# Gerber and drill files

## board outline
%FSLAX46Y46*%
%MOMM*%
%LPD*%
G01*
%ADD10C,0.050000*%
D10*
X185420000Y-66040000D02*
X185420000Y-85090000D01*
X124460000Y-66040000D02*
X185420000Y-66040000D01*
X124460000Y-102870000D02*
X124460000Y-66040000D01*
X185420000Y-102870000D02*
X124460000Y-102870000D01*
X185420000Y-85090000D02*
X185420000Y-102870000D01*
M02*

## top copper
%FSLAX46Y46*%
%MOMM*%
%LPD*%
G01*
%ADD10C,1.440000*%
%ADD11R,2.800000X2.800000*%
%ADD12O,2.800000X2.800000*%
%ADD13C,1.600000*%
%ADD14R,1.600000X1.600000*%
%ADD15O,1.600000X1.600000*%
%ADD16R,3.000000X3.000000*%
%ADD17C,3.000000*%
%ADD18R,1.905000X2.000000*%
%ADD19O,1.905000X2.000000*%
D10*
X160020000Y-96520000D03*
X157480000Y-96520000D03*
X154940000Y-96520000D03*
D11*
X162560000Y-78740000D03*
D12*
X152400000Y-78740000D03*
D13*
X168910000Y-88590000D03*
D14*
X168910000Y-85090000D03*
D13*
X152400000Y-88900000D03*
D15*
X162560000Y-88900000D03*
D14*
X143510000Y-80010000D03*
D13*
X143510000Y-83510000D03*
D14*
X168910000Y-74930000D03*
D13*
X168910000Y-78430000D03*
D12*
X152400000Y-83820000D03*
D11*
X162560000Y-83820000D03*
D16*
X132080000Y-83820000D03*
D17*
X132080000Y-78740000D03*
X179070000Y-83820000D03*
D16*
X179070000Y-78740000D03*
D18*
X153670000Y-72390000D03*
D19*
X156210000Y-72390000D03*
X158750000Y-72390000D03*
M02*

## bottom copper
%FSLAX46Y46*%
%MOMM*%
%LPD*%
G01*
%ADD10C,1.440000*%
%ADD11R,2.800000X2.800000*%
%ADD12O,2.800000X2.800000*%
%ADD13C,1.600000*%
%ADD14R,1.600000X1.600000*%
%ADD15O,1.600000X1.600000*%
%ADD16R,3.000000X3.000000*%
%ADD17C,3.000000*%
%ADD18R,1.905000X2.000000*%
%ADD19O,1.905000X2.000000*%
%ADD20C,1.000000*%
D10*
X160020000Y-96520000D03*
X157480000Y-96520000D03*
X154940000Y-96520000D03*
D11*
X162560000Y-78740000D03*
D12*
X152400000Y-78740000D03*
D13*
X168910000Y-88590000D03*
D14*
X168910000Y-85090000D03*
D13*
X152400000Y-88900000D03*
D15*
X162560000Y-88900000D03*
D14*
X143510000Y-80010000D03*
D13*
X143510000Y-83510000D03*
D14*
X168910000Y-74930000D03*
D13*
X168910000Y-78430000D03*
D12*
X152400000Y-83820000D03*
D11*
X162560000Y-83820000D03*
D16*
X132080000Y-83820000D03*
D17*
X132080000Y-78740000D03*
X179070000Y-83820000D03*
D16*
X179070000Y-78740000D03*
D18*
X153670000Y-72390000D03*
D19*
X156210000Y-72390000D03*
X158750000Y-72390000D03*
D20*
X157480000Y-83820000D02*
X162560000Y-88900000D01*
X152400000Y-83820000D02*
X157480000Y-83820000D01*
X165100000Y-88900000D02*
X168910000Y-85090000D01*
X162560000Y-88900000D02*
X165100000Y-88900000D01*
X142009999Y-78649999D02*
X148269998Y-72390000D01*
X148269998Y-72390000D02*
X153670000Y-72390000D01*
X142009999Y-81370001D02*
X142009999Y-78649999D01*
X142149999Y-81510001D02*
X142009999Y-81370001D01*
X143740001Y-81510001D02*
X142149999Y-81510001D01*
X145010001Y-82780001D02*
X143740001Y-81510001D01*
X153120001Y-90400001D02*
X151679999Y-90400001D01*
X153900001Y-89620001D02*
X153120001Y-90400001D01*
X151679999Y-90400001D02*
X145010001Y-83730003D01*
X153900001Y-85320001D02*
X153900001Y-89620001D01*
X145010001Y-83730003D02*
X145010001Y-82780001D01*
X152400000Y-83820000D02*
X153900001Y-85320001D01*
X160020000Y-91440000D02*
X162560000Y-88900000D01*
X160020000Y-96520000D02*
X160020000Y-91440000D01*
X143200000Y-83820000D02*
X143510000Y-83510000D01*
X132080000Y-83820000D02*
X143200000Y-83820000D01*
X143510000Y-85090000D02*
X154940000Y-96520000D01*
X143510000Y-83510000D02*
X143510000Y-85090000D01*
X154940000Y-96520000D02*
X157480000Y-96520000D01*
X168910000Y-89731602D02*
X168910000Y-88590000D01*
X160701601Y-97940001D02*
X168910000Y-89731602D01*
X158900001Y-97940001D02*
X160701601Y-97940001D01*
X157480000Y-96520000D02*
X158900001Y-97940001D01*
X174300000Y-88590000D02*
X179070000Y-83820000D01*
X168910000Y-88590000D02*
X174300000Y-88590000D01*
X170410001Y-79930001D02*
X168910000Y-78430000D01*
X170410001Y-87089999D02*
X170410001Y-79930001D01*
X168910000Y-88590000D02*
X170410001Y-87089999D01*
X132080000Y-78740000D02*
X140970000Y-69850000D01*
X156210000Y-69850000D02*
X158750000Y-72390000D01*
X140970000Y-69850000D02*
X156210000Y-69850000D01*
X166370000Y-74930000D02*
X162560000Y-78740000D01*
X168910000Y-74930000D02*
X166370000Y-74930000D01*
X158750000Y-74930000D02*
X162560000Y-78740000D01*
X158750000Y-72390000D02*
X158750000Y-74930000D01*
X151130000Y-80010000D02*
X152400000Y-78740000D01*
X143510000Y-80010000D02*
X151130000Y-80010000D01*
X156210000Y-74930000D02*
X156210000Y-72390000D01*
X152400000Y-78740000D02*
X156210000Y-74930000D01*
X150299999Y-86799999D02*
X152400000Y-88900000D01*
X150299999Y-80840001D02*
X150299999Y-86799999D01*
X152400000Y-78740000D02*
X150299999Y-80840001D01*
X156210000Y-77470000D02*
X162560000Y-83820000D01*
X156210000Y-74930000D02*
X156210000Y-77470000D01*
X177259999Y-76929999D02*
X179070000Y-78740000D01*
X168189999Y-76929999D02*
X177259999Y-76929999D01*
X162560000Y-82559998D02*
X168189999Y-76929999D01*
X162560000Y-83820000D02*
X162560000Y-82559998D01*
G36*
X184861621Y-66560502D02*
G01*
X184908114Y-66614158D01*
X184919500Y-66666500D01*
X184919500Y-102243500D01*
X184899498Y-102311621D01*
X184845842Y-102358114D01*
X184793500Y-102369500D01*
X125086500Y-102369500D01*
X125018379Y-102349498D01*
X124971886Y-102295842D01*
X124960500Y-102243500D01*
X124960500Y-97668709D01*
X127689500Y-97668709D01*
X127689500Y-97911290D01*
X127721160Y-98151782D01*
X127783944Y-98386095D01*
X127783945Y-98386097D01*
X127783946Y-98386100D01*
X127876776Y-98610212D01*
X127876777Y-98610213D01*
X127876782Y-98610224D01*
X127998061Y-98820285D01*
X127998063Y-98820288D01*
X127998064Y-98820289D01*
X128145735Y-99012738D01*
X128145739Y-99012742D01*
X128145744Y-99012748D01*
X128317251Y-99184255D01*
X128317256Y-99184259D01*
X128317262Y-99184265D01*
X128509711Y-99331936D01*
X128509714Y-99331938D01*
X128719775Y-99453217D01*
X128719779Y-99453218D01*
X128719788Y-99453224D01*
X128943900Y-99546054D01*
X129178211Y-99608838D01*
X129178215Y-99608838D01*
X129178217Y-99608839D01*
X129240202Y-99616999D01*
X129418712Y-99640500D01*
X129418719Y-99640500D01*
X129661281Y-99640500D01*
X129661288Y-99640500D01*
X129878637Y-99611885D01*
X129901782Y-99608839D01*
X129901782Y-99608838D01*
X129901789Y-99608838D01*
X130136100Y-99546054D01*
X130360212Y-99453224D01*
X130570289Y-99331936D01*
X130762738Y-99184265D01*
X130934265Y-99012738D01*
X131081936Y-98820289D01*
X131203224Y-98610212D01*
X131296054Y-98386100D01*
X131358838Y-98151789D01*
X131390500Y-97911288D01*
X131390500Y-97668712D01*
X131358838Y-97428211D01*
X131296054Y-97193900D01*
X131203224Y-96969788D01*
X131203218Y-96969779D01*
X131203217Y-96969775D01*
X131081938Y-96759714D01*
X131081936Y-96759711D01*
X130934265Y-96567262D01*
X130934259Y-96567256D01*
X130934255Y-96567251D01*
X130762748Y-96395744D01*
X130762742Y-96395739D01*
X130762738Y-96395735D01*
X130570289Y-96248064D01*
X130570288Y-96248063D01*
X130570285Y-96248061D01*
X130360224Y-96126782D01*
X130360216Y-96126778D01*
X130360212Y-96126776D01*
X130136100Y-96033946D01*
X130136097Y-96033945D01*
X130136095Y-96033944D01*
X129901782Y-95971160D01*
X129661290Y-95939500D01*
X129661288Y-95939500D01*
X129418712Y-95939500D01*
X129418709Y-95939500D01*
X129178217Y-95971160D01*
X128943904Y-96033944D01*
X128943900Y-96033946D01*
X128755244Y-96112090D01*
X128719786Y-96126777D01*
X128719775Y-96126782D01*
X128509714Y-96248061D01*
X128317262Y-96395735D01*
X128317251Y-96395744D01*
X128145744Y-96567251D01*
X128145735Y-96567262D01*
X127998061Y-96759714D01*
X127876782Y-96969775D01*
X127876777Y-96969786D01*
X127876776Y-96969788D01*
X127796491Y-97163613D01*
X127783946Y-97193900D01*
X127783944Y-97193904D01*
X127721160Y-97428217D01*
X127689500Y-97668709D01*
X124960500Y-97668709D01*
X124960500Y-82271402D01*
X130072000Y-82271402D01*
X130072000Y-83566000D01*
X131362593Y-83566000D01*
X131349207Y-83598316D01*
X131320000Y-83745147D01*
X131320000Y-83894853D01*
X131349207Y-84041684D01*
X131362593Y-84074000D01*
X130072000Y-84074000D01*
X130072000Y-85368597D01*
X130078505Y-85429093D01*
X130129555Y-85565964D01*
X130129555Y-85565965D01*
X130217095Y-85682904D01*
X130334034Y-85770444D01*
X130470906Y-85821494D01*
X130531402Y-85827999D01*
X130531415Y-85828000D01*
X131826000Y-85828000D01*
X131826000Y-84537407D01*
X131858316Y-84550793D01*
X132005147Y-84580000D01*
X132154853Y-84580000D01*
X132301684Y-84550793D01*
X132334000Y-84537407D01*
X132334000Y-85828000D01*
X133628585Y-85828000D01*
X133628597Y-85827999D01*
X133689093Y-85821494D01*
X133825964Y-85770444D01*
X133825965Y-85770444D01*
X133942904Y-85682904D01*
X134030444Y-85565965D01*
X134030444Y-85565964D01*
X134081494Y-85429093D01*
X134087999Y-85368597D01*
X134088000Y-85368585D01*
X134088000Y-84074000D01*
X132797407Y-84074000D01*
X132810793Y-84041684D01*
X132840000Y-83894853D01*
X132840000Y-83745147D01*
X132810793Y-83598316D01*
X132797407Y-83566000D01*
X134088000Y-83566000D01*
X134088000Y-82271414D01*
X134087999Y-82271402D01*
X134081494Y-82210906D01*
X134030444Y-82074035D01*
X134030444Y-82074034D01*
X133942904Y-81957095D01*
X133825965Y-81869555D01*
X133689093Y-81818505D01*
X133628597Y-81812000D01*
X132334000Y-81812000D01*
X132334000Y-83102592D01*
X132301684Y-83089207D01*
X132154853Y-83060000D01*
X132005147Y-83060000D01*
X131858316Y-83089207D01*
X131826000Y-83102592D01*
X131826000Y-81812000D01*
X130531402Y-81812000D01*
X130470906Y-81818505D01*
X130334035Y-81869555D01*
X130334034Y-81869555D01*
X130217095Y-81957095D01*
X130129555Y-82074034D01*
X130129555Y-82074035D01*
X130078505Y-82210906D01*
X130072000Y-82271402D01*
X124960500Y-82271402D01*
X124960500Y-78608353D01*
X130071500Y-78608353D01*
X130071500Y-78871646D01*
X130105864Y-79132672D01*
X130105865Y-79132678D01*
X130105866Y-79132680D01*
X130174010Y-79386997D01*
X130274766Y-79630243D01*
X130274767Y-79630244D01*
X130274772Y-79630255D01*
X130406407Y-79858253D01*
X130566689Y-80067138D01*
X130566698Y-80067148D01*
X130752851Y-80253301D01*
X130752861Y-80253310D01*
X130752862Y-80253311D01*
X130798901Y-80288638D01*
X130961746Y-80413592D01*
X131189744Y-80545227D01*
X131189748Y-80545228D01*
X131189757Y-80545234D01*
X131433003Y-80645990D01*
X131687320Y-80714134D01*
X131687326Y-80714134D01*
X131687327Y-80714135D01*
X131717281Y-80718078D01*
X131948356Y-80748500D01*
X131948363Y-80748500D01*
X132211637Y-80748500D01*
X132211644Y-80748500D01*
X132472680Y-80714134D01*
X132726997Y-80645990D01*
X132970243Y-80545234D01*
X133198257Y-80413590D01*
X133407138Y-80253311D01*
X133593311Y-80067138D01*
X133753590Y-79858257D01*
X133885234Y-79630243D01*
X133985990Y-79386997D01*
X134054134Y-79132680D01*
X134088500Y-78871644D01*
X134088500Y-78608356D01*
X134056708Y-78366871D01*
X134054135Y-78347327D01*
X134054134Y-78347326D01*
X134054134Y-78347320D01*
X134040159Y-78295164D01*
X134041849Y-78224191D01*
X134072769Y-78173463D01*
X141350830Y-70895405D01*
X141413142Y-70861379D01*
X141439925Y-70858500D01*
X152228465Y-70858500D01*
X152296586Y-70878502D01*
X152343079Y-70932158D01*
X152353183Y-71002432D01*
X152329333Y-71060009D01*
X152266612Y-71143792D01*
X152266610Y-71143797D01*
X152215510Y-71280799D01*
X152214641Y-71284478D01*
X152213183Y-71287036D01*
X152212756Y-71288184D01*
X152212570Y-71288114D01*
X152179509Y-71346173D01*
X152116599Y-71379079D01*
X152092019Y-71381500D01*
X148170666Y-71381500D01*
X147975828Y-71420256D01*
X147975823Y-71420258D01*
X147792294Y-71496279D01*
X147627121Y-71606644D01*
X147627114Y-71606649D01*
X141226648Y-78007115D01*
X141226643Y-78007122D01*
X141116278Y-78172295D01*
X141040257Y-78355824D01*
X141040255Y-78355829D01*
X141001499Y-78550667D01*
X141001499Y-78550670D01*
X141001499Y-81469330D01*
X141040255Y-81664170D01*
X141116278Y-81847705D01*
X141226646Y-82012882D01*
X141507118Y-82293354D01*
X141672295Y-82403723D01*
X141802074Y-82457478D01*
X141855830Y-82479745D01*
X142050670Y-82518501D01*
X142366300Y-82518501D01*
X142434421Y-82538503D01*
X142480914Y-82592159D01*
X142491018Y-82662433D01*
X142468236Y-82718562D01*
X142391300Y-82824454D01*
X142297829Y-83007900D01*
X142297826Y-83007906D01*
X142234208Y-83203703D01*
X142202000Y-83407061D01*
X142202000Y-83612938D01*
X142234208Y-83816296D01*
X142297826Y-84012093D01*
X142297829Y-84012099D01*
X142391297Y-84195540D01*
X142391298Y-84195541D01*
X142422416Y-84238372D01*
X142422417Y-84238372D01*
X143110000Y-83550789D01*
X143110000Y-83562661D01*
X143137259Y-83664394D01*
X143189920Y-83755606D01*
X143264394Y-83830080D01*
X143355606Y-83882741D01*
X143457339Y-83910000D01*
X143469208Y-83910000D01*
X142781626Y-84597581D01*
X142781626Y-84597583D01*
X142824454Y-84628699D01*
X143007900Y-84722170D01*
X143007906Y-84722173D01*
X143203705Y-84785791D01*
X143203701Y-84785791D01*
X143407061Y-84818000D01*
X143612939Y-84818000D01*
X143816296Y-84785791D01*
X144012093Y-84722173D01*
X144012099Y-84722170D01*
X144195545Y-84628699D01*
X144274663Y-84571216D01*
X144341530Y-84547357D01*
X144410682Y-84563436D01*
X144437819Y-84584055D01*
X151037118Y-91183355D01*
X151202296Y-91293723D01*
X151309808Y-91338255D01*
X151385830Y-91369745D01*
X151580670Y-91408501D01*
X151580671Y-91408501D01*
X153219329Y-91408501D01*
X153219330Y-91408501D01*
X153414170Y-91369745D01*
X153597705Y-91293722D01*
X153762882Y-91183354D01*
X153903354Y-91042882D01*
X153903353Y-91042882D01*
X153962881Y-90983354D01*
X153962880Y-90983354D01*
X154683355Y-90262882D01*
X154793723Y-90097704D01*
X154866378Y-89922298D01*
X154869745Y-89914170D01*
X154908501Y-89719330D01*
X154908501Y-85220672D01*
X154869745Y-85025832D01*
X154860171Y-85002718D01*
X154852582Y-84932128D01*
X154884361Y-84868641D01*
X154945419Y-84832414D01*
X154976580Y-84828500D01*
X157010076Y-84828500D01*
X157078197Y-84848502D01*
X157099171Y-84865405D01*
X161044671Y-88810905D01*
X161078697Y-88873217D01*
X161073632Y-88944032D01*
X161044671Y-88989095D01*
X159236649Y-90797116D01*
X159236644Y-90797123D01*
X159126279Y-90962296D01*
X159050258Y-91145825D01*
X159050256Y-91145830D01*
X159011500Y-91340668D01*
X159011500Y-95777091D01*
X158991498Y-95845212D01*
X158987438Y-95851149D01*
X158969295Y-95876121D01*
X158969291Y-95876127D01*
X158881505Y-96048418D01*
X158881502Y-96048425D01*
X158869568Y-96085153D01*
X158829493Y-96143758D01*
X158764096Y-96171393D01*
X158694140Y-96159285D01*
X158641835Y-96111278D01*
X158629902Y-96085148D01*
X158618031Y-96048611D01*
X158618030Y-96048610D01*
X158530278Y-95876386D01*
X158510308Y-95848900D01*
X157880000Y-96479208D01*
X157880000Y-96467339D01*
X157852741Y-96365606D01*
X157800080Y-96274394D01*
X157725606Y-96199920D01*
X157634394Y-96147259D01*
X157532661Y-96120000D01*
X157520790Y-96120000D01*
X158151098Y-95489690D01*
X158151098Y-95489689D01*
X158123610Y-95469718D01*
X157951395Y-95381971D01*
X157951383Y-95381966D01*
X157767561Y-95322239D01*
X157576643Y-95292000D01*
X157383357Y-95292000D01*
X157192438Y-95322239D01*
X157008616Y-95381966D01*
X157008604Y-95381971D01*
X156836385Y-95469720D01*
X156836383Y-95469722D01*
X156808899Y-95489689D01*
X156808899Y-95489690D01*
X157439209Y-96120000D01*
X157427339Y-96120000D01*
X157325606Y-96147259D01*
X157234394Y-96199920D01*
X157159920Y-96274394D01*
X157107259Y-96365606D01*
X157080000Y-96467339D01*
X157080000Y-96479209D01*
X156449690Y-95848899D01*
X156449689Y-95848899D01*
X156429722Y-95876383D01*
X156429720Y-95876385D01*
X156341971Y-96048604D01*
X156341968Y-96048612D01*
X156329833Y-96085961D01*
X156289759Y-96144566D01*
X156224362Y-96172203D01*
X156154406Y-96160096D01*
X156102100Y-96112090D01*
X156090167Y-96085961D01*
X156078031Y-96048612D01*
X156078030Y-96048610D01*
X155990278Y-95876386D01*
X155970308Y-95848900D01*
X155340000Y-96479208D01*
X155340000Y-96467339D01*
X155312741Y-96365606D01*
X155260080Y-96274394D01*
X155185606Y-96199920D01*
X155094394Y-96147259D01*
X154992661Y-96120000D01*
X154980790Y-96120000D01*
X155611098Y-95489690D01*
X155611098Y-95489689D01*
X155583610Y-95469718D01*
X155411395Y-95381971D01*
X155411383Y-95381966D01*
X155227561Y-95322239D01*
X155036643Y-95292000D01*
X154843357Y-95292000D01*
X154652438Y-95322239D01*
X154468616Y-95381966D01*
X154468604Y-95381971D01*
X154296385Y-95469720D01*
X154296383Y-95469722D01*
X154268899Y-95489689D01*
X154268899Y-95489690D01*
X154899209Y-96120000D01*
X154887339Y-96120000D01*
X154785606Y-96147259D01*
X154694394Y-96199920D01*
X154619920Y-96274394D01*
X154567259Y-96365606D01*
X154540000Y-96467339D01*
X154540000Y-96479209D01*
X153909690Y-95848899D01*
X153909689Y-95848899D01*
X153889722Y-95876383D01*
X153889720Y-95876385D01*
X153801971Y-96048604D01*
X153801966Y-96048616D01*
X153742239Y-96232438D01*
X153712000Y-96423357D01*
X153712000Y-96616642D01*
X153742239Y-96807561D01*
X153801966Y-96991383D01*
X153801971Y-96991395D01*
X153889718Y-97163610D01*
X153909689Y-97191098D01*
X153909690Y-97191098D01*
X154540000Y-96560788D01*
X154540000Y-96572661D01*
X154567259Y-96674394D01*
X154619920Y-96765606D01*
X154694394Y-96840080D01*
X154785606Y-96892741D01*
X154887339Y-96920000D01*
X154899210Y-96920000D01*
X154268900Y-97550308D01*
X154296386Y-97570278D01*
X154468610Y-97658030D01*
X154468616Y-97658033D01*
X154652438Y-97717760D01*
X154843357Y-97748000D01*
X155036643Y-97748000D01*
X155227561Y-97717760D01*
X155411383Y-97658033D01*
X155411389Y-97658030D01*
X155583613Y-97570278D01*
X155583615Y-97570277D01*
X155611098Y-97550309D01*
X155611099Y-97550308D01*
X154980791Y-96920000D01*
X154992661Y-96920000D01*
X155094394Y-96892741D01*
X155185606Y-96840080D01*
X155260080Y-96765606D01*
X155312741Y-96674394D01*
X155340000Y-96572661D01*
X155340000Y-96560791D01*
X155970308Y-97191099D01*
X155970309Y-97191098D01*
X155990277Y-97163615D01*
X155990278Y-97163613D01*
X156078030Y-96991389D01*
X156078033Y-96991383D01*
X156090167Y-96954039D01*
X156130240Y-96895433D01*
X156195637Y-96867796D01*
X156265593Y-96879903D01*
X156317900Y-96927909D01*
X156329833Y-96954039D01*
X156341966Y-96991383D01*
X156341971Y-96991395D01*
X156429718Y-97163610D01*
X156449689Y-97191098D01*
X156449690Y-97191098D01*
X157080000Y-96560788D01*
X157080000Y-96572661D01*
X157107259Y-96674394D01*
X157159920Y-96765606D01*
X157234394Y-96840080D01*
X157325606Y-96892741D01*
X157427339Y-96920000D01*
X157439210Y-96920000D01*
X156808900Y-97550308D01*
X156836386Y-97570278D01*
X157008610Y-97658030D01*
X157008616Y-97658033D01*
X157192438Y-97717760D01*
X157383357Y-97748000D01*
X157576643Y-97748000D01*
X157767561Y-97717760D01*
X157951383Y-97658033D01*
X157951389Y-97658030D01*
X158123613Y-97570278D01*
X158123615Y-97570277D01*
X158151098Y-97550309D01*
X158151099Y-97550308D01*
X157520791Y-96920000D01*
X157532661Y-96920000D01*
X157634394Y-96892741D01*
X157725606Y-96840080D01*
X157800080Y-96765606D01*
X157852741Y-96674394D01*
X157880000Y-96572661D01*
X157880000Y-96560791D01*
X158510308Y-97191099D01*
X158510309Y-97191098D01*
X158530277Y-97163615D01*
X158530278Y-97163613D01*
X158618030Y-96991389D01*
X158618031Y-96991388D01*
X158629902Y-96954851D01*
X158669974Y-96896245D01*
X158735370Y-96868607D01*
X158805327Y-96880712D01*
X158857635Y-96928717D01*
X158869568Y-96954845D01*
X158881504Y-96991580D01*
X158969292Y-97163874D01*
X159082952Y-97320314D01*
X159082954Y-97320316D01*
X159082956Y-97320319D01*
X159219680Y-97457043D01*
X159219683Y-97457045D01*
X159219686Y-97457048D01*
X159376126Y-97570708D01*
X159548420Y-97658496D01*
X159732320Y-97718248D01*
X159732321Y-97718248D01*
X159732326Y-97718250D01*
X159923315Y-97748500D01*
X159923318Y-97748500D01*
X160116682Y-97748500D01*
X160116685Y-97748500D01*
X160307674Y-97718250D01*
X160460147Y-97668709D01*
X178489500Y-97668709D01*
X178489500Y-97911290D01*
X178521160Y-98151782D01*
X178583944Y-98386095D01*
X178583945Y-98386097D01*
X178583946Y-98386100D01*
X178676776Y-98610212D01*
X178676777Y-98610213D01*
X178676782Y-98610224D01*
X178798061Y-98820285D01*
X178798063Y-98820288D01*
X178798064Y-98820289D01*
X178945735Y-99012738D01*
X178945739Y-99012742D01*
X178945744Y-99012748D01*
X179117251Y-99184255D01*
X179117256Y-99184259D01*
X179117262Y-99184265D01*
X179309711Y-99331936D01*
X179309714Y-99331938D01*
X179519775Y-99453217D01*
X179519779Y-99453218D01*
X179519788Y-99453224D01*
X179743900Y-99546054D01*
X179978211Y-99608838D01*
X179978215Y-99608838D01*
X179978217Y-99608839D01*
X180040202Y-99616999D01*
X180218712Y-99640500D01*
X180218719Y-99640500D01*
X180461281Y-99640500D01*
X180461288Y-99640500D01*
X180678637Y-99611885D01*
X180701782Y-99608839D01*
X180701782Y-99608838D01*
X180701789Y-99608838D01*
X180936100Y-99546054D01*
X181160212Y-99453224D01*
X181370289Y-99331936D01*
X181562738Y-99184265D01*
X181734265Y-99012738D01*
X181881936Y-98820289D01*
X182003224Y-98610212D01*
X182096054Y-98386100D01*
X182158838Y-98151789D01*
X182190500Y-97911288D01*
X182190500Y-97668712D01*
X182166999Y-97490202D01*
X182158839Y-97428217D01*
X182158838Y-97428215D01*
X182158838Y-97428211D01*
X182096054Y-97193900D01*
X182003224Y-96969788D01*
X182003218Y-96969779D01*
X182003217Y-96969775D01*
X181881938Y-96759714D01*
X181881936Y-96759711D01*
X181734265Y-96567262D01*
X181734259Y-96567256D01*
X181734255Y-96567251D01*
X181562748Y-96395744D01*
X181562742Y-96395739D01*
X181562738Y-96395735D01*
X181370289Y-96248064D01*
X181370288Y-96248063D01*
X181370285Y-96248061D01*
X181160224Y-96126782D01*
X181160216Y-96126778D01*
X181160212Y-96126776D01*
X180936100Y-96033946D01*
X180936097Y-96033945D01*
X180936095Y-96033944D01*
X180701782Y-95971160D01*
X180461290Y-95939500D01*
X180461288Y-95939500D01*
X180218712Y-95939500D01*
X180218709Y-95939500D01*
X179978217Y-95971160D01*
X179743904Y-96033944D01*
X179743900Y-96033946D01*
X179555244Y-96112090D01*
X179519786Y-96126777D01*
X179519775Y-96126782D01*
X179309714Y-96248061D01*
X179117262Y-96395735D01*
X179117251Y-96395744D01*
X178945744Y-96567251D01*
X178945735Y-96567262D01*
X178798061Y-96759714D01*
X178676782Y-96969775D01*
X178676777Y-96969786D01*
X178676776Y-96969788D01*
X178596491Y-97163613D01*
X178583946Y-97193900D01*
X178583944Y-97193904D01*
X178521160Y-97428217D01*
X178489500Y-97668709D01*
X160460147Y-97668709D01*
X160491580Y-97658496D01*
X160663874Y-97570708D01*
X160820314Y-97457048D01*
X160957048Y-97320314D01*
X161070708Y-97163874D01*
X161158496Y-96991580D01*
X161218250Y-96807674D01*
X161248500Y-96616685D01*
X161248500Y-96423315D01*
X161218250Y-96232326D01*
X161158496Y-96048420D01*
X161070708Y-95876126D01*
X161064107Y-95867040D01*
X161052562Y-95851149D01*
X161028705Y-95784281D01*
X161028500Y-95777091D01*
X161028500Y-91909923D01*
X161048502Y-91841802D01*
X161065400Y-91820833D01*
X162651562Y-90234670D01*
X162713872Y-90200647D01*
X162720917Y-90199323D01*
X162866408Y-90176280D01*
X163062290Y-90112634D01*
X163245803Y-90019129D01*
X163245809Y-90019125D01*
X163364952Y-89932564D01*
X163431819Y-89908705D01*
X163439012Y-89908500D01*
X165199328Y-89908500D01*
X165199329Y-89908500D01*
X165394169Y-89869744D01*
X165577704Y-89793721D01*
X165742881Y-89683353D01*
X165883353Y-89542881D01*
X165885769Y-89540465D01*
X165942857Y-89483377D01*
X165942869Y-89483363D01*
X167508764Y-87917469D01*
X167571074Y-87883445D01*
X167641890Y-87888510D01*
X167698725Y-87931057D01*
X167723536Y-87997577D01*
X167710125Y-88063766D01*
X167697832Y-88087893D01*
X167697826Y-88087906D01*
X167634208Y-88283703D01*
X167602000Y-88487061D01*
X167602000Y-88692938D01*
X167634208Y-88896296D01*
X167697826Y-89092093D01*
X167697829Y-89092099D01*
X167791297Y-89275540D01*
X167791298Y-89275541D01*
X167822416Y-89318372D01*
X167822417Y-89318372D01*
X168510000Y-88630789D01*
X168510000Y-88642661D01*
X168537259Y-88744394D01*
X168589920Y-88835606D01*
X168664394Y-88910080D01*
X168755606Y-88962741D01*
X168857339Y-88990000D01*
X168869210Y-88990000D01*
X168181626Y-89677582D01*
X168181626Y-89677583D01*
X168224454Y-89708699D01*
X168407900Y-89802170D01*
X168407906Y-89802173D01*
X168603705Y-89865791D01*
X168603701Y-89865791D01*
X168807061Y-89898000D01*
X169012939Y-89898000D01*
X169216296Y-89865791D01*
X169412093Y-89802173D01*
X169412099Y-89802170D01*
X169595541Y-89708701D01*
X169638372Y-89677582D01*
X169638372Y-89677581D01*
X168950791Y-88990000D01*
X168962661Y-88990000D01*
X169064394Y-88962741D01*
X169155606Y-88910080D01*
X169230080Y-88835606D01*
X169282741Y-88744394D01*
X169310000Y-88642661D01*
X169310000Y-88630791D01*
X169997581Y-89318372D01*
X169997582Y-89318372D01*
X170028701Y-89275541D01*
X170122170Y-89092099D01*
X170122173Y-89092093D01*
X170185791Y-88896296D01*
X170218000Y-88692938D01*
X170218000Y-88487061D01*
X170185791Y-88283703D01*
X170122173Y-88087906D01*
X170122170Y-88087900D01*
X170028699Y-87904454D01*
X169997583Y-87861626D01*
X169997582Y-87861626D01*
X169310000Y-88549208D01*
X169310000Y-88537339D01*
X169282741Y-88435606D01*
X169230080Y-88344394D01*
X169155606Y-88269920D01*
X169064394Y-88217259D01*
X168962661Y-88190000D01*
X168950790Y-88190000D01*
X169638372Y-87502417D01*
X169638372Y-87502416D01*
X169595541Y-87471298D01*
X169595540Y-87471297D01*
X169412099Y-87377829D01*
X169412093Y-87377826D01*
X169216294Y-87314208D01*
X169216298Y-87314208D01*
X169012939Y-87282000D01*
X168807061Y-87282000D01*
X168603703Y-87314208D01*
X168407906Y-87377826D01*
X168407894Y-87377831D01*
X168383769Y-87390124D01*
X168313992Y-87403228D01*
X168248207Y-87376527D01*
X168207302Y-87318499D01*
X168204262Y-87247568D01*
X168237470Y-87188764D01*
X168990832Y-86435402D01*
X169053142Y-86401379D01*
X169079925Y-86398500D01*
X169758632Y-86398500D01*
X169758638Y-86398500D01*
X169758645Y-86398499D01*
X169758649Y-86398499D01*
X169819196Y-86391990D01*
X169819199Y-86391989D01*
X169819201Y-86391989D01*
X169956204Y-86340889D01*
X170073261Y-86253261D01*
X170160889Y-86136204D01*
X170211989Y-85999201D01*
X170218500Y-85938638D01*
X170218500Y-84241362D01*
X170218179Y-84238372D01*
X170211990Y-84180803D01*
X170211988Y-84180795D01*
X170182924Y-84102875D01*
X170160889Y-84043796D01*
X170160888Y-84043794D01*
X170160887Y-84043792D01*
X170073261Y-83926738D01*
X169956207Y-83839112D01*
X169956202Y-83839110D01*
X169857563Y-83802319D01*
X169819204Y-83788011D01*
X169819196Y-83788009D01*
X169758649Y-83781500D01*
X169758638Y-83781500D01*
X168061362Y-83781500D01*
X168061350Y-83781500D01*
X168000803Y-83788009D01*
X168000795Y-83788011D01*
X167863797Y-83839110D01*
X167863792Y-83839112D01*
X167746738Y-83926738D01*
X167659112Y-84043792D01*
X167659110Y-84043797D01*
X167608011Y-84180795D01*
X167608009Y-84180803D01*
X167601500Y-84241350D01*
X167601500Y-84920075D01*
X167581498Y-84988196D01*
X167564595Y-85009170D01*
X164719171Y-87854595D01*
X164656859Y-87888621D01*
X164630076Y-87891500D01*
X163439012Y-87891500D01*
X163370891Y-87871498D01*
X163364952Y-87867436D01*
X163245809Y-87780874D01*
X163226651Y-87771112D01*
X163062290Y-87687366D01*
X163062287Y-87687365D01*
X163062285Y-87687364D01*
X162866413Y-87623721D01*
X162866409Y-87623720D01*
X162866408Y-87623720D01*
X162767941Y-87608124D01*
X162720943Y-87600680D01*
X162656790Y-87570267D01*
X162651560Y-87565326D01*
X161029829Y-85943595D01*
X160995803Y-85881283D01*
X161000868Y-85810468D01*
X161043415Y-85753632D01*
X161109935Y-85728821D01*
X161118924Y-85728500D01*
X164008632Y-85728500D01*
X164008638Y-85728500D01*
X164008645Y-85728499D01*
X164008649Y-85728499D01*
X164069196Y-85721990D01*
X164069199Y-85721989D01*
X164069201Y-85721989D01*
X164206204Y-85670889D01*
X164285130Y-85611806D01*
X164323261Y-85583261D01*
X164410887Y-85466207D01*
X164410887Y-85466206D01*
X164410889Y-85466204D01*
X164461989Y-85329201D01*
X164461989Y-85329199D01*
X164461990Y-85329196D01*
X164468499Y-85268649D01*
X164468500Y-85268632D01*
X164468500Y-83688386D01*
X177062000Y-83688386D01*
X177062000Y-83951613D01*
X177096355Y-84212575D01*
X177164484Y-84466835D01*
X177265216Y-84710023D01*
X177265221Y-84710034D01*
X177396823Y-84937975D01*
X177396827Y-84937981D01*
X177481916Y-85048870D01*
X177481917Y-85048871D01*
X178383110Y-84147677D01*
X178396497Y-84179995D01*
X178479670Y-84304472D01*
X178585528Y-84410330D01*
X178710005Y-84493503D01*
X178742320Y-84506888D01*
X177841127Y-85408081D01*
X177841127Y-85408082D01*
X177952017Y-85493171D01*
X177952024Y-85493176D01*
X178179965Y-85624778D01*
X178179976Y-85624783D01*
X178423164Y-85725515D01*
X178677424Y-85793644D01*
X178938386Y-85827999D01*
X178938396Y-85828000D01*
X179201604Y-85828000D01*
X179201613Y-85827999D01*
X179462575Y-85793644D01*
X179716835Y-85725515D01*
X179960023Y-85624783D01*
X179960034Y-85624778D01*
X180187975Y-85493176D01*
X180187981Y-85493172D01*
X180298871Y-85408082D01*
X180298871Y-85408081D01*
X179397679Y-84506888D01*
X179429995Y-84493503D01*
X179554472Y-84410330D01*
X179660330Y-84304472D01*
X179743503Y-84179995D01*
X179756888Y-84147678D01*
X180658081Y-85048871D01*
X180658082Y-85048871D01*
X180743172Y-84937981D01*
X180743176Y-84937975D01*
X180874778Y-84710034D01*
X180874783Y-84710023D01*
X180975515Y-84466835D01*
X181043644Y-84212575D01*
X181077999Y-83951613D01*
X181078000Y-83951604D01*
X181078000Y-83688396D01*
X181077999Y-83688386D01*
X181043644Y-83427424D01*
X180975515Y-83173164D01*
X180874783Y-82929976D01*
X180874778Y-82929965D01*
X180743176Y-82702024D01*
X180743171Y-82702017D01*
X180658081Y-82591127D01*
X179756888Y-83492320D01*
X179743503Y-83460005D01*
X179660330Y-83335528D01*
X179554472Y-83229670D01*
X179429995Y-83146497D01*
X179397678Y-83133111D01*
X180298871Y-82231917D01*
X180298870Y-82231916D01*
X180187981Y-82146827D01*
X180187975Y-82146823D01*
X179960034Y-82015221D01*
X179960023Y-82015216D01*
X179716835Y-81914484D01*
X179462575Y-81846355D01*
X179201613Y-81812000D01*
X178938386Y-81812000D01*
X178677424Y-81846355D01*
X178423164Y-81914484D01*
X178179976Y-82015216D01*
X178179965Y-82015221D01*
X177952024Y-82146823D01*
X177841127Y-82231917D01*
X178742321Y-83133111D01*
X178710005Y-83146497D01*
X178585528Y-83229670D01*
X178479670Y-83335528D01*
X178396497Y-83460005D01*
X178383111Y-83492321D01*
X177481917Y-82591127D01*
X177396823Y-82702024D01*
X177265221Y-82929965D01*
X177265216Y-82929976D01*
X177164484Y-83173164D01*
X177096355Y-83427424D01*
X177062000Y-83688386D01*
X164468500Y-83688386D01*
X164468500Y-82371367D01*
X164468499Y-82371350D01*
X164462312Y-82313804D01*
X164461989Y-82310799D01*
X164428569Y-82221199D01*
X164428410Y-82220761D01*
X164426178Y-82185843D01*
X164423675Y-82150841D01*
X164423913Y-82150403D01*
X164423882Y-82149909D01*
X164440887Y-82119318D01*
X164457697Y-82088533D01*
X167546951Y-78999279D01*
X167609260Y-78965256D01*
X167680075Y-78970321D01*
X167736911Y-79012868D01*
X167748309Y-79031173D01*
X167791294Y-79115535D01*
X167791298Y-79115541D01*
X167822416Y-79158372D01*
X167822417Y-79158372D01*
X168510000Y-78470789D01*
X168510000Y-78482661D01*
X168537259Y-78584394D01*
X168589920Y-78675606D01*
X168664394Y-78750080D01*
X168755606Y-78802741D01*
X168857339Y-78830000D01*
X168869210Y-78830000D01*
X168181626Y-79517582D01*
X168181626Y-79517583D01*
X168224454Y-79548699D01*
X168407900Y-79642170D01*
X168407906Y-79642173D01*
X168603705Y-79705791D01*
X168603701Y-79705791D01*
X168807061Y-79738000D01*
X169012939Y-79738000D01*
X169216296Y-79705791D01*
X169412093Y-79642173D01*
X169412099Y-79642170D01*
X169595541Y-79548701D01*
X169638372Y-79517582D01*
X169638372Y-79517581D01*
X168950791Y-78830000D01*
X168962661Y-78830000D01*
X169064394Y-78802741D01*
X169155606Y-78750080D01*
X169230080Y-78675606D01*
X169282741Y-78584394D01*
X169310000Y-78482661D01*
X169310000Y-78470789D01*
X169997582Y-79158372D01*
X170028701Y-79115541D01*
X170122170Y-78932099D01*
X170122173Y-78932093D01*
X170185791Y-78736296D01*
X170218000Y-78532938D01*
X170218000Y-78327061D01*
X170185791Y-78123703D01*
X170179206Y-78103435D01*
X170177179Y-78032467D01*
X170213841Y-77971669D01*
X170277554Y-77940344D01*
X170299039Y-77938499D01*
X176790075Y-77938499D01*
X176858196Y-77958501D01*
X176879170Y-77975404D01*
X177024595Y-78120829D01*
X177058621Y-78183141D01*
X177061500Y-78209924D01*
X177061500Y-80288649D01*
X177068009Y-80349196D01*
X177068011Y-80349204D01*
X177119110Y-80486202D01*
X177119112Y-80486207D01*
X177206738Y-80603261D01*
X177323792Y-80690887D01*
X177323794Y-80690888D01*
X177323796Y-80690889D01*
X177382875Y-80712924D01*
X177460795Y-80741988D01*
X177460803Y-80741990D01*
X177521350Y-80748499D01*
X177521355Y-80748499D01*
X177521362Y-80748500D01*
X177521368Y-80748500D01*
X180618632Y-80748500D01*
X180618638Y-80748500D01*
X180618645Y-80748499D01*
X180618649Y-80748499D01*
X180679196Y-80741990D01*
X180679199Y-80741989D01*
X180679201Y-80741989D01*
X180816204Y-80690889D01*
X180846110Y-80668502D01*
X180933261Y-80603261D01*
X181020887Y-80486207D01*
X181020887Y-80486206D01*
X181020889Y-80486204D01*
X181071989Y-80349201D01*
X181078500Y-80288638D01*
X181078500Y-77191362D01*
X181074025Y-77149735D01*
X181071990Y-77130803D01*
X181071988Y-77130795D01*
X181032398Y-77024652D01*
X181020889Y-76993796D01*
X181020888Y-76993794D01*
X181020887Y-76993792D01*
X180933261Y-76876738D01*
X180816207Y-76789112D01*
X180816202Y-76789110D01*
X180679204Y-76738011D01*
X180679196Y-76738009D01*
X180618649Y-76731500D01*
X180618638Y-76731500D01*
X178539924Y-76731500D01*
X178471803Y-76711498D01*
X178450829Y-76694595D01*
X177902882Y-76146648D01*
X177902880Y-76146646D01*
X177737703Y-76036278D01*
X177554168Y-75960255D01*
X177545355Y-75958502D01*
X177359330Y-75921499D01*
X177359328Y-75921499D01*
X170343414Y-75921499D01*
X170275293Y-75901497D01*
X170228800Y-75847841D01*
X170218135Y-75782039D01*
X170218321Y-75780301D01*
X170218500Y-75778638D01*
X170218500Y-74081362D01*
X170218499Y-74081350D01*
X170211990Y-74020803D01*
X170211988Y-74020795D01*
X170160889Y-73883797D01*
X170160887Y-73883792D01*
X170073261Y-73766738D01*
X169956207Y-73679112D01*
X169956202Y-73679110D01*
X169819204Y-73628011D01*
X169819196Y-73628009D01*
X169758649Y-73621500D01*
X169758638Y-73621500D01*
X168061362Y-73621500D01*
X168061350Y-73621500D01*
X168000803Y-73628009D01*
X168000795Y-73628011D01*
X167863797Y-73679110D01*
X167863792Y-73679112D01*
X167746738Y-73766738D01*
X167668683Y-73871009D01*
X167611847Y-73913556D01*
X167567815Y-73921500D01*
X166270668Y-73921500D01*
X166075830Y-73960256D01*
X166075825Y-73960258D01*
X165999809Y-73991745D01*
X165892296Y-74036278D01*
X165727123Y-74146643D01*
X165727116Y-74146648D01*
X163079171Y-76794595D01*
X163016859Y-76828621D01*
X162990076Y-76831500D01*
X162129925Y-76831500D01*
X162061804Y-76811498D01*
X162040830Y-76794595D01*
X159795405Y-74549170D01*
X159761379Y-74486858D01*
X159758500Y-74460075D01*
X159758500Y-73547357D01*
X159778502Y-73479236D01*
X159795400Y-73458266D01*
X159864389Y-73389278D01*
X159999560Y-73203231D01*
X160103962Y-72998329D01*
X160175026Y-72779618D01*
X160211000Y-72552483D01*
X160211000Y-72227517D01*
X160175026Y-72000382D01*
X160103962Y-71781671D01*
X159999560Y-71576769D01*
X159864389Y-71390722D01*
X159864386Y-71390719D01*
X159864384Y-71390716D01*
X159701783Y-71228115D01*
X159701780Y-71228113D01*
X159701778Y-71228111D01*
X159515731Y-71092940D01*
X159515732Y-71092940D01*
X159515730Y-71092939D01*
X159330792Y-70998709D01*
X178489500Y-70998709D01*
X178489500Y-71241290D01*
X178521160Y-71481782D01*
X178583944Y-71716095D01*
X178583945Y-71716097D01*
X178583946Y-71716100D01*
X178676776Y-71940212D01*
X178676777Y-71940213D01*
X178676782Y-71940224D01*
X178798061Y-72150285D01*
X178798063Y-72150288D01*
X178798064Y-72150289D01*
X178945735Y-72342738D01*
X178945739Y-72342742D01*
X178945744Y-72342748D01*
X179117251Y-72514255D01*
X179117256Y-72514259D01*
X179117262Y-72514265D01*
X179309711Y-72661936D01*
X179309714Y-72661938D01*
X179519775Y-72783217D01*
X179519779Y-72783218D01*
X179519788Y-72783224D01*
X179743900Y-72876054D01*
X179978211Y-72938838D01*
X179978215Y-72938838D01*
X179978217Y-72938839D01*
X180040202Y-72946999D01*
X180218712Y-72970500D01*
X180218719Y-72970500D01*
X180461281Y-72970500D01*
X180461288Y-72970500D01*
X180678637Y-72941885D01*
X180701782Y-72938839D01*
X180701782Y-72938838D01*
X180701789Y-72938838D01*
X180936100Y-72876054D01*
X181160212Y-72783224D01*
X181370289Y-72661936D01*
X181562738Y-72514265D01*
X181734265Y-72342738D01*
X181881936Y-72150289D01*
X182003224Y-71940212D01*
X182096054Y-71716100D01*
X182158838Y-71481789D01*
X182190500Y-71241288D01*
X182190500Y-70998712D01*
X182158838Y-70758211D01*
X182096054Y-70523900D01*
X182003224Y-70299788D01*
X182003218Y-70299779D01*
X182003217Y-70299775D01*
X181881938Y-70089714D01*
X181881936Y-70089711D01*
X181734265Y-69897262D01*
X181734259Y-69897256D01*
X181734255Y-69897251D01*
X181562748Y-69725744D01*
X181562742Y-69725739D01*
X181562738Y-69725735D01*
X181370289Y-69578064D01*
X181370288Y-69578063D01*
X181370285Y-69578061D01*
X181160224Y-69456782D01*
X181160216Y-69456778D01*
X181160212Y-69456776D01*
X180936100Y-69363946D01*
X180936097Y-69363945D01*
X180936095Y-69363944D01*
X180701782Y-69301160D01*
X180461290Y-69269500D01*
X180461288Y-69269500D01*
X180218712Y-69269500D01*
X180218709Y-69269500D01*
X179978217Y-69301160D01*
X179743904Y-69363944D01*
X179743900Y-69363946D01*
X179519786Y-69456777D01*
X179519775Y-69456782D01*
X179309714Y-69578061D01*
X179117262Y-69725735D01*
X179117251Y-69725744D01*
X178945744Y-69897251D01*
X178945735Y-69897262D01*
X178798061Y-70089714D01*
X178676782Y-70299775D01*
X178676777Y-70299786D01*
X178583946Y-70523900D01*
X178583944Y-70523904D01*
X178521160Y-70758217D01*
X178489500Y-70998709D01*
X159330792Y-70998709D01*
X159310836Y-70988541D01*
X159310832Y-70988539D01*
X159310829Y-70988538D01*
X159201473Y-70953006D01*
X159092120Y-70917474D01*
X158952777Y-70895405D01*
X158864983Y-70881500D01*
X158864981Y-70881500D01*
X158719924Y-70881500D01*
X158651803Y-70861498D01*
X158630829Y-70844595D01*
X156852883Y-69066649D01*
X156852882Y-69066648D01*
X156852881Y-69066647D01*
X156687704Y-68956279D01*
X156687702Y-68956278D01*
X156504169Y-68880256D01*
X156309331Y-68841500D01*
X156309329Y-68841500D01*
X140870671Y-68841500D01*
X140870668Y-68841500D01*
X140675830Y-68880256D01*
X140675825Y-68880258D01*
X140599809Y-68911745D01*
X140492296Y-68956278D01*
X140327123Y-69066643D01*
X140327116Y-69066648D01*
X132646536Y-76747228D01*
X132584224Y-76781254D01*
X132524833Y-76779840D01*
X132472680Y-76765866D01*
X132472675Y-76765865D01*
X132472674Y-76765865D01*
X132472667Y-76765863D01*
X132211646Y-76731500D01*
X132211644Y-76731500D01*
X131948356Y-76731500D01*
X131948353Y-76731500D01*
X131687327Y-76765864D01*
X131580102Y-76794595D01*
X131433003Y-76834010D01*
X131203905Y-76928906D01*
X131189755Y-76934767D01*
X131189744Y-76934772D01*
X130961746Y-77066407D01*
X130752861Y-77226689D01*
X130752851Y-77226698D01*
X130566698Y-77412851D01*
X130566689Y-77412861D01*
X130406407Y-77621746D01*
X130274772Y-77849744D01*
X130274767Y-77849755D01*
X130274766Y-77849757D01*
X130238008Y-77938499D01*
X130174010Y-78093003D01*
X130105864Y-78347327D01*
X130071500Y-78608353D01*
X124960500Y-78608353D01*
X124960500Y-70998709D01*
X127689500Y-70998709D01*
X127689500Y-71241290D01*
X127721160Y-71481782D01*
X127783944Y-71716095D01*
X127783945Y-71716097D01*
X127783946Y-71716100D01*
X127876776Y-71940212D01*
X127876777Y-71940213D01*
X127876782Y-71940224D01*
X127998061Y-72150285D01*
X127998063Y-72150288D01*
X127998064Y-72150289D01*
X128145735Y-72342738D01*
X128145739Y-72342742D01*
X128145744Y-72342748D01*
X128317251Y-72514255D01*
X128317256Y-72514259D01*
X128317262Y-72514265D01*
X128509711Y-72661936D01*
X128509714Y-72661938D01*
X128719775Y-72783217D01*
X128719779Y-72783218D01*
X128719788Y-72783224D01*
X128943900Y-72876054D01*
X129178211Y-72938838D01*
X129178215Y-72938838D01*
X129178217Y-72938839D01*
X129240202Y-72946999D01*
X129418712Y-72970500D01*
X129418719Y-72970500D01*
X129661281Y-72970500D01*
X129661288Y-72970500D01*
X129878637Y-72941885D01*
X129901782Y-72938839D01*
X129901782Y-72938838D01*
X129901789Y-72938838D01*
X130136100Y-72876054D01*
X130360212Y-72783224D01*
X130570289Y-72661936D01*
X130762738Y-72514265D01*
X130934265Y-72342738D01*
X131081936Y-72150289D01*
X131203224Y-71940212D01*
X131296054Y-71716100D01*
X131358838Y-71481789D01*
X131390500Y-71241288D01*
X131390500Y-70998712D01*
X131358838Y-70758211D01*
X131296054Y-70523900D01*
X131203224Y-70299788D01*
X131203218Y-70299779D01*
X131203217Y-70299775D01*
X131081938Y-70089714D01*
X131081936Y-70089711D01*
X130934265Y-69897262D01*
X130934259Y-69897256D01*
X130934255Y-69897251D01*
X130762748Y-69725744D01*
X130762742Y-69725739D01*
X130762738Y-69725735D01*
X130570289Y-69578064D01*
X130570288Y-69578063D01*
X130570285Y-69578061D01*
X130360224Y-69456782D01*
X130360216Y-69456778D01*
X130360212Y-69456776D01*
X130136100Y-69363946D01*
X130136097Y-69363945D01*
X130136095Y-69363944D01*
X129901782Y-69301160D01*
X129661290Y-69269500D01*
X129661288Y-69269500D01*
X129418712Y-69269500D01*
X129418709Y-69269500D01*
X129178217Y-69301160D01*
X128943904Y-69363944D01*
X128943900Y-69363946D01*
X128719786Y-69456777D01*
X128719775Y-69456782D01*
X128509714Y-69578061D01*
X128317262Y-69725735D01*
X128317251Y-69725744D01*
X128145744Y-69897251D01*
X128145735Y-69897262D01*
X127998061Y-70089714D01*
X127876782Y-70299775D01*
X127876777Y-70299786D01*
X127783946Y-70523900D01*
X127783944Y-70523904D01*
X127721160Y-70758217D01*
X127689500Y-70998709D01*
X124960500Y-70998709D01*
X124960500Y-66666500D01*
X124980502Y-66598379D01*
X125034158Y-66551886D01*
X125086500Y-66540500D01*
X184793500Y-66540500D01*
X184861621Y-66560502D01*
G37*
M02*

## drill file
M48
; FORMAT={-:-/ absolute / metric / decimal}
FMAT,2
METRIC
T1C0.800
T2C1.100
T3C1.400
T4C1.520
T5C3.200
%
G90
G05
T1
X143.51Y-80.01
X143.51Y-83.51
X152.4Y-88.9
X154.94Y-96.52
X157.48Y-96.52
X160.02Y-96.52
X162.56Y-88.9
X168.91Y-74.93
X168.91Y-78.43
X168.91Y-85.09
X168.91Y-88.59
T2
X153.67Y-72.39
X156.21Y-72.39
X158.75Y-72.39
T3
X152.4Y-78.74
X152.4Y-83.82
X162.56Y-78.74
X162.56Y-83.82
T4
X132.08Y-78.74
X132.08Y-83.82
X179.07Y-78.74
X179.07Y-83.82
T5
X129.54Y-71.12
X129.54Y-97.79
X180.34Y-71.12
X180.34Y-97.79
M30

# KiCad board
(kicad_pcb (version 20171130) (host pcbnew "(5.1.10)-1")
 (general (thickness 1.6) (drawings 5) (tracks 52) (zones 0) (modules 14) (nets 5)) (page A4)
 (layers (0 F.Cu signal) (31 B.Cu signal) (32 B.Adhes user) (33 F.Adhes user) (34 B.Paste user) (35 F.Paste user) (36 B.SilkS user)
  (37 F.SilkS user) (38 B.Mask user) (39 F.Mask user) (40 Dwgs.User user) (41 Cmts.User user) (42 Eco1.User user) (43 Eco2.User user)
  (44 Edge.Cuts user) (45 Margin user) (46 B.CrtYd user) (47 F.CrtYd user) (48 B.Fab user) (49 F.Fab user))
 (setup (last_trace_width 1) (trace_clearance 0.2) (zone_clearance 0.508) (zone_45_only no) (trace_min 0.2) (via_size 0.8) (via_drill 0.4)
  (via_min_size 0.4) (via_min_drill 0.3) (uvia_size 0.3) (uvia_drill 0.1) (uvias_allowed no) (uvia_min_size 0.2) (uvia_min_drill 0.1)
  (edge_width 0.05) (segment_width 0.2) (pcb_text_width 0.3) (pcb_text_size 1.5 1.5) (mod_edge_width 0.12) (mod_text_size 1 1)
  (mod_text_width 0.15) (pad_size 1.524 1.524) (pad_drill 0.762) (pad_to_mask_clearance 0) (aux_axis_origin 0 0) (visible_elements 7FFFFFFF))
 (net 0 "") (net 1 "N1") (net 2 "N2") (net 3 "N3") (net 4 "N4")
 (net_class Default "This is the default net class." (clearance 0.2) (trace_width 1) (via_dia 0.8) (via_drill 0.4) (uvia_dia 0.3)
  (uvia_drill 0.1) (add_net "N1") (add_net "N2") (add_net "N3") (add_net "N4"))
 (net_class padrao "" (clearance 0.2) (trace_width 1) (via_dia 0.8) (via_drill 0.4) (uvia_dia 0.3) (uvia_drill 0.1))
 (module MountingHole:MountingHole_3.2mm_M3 (layer F.Cu) (at 129.54 97.79)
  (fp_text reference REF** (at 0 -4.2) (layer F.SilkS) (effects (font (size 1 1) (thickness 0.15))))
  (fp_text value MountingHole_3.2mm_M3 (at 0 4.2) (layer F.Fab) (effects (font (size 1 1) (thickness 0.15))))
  (pad 1 np_thru_hole circle (at 0 0) (size 3.2 3.2) (drill 3.2) (layers *.Cu *.Mask)))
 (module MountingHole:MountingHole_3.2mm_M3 (layer F.Cu) (at 129.54 71.12)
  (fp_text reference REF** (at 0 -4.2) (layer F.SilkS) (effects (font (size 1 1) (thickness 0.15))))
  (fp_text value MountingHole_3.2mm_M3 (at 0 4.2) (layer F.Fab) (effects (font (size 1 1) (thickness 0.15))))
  (pad 1 np_thru_hole circle (at 0 0) (size 3.2 3.2) (drill 3.2) (layers *.Cu *.Mask)))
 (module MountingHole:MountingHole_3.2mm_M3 (layer F.Cu) (at 180.34 97.79)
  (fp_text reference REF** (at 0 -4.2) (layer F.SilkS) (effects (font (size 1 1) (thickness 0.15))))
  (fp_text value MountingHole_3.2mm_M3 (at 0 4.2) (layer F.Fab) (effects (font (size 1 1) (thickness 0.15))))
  (pad 1 np_thru_hole circle (at 0 0) (size 3.2 3.2) (drill 3.2) (layers *.Cu *.Mask)))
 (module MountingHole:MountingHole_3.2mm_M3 (layer F.Cu) (at 180.34 71.12)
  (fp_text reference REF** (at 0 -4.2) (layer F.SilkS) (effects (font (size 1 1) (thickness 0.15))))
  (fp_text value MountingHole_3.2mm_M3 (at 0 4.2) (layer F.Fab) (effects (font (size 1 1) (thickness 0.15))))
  (pad 1 np_thru_hole circle (at 0 0) (size 3.2 3.2) (drill 3.2) (layers *.Cu *.Mask)))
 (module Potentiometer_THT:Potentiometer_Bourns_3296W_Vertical (layer F.Cu) (at 160.02 96.52)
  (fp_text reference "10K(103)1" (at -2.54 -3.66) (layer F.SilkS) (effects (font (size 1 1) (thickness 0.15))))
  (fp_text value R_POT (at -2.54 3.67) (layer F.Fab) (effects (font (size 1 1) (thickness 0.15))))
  (pad 1 thru_hole circle (at 0 0) (size 1.44 1.44) (drill 0.8) (layers *.Cu *.Mask) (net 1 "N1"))
  (pad 2 thru_hole circle (at -2.54 0) (size 1.44 1.44) (drill 0.8) (layers *.Cu *.Mask) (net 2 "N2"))
  (pad 3 thru_hole circle (at -5.08 0) (size 1.44 1.44) (drill 0.8) (layers *.Cu *.Mask) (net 2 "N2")))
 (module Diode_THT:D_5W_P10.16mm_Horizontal (layer F.Cu) (at 162.56 78.74 180)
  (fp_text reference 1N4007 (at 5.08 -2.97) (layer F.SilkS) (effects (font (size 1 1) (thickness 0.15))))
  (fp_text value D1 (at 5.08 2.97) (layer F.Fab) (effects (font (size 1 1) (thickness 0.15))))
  (pad 1 thru_hole rect (at 0 0 180) (size 2.8 2.8) (drill 1.4) (layers *.Cu *.Mask) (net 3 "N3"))
  (pad 2 thru_hole oval (at 10.16 0 180) (size 2.8 2.8) (drill 1.4) (layers *.Cu *.Mask) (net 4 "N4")))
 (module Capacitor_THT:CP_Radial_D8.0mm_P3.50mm (layer F.Cu) (at 168.91 85.09 270)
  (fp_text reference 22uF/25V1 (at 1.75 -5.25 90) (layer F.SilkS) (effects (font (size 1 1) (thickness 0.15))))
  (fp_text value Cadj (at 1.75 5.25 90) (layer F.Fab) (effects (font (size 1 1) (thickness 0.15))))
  (pad 2 thru_hole circle (at 3.5 0 270) (size 1.6 1.6) (drill 0.8) (layers *.Cu *.Mask) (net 2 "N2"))
  (pad 1 thru_hole rect (at 0 0 270) (size 1.6 1.6) (drill 0.8) (layers *.Cu *.Mask) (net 1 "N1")))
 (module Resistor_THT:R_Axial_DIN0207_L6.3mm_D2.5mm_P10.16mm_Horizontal (layer F.Cu) (at 152.4 88.9)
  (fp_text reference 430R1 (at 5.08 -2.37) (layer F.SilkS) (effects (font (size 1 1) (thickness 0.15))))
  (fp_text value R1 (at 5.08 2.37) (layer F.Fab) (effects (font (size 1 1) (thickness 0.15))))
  (pad 1 thru_hole circle (at 0 0) (size 1.6 1.6) (drill 0.8) (layers *.Cu *.Mask) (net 4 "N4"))
  (pad 2 thru_hole oval (at 10.16 0) (size 1.6 1.6) (drill 0.8) (layers *.Cu *.Mask) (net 1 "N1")))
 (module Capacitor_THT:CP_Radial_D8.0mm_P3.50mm (layer F.Cu) (at 143.51 80.01 270)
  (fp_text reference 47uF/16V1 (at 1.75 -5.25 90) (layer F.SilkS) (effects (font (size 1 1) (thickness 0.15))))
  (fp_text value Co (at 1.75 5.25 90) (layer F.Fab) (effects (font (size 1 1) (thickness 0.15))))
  (pad 1 thru_hole rect (at 0 0 270) (size 1.6 1.6) (drill 0.8) (layers *.Cu *.Mask) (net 4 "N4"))
  (pad 2 thru_hole circle (at 3.5 0 270) (size 1.6 1.6) (drill 0.8) (layers *.Cu *.Mask) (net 2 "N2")))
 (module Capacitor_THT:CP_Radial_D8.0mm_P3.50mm (layer F.Cu) (at 168.91 74.93 270)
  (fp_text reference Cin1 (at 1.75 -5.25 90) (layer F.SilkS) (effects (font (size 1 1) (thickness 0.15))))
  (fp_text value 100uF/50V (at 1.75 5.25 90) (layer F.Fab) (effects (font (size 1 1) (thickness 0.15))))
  (pad 1 thru_hole rect (at 0 0 270) (size 1.6 1.6) (drill 0.8) (layers *.Cu *.Mask) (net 3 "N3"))
  (pad 2 thru_hole circle (at 3.5 0 270) (size 1.6 1.6) (drill 0.8) (layers *.Cu *.Mask) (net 2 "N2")))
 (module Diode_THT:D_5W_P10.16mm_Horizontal (layer F.Cu) (at 162.56 83.82 180)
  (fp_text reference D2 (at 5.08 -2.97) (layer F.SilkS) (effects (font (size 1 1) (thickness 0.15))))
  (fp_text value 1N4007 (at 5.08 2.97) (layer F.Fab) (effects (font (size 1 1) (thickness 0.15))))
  (pad 2 thru_hole oval (at 10.16 0 180) (size 2.8 2.8) (drill 1.4) (layers *.Cu *.Mask) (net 1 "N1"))
  (pad 1 thru_hole rect (at 0 0 180) (size 2.8 2.8) (drill 1.4) (layers *.Cu *.Mask) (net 4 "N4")))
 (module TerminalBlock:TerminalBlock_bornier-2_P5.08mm (layer F.Cu) (at 132.08 83.82 90)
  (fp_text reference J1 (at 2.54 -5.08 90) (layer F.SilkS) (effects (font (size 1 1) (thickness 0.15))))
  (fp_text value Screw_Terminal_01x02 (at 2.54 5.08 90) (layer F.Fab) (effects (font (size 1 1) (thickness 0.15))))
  (pad 1 thru_hole rect (at 0 0 90) (size 3 3) (drill 1.52) (layers *.Cu *.Mask) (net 2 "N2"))
  (pad 2 thru_hole circle (at 5.08 0 90) (size 3 3) (drill 1.52) (layers *.Cu *.Mask) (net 3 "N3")))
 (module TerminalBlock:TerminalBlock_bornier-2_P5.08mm (layer F.Cu) (at 179.07 78.74 270)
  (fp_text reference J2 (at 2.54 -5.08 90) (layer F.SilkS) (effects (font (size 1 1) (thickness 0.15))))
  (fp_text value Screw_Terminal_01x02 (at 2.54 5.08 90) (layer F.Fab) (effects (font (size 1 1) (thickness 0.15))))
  (pad 2 thru_hole circle (at 5.08 0 270) (size 3 3) (drill 1.52) (layers *.Cu *.Mask) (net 2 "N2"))
  (pad 1 thru_hole rect (at 0 0 270) (size 3 3) (drill 1.52) (layers *.Cu *.Mask) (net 4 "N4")))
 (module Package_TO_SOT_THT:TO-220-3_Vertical (layer F.Cu) (at 153.67 72.39)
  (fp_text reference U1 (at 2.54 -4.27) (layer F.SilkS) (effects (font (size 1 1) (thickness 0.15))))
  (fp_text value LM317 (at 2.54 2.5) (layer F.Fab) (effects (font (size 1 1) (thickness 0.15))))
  (pad 1 thru_hole rect (at 0 0) (size 1.905 2) (drill 1.1) (layers *.Cu *.Mask) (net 1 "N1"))
  (pad 2 thru_hole oval (at 2.54 0) (size 1.905 2) (drill 1.1) (layers *.Cu *.Mask) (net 4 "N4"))
  (pad 3 thru_hole oval (at 5.08 0) (size 1.905 2) (drill 1.1) (layers *.Cu *.Mask) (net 3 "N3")))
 (gr_line (start 185.42 66.04) (end 185.42 85.09) (layer Edge.Cuts) (width 0.05))
 (gr_line (start 124.46 66.04) (end 185.42 66.04) (layer Edge.Cuts) (width 0.05))
 (gr_line (start 124.46 102.87) (end 124.46 66.04) (layer Edge.Cuts) (width 0.05))
 (gr_line (start 185.42 102.87) (end 124.46 102.87) (layer Edge.Cuts) (width 0.05))
 (gr_line (start 185.42 85.09) (end 185.42 102.87) (layer Edge.Cuts) (width 0.05))
 (segment (start 157.48 83.82) (end 162.56 88.9) (width 1) (layer B.Cu) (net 1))
 (segment (start 152.4 83.82) (end 157.48 83.82) (width 1) (layer B.Cu) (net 1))
 (segment (start 165.1 88.9) (end 168.91 85.09) (width 1) (layer B.Cu) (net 1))
 (segment (start 162.56 88.9) (end 165.1 88.9) (width 1) (layer B.Cu) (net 1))
 (segment (start 142.009999 78.649999) (end 148.269998 72.39) (width 1) (layer B.Cu) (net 1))
 (segment (start 148.269998 72.39) (end 153.67 72.39) (width 1) (layer B.Cu) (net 1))
 (segment (start 142.009999 81.370001) (end 142.009999 78.649999) (width 1) (layer B.Cu) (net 1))
 (segment (start 142.149999 81.510001) (end 142.009999 81.370001) (width 1) (layer B.Cu) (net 1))
 (segment (start 143.740001 81.510001) (end 142.149999 81.510001) (width 1) (layer B.Cu) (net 1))
 (segment (start 145.010001 82.780001) (end 143.740001 81.510001) (width 1) (layer B.Cu) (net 1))
 (segment (start 153.120001 90.400001) (end 151.679999 90.400001) (width 1) (layer B.Cu) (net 1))
 (segment (start 153.900001 89.620001) (end 153.120001 90.400001) (width 1) (layer B.Cu) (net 1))
 (segment (start 151.679999 90.400001) (end 145.010001 83.730003) (width 1) (layer B.Cu) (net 1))
 (segment (start 153.900001 85.320001) (end 153.900001 89.620001) (width 1) (layer B.Cu) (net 1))
 (segment (start 145.010001 83.730003) (end 145.010001 82.780001) (width 1) (layer B.Cu) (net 1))
 (segment (start 152.4 83.82) (end 153.900001 85.320001) (width 1) (layer B.Cu) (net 1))
 (segment (start 160.02 91.44) (end 162.56 88.9) (width 1) (layer B.Cu) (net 1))
 (segment (start 160.02 96.52) (end 160.02 91.44) (width 1) (layer B.Cu) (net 1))
 (segment (start 143.2 83.82) (end 143.51 83.51) (width 1) (layer B.Cu) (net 2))
 (segment (start 132.08 83.82) (end 143.2 83.82) (width 1) (layer B.Cu) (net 2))
 (segment (start 143.51 85.09) (end 154.94 96.52) (width 1) (layer B.Cu) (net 2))
 (segment (start 143.51 83.51) (end 143.51 85.09) (width 1) (layer B.Cu) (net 2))
 (segment (start 154.94 96.52) (end 157.48 96.52) (width 1) (layer B.Cu) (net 2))
 (segment (start 168.91 89.731602) (end 168.91 88.59) (width 1) (layer B.Cu) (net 2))
 (segment (start 160.701601 97.940001) (end 168.91 89.731602) (width 1) (layer B.Cu) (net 2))
 (segment (start 158.900001 97.940001) (end 160.701601 97.940001) (width 1) (layer B.Cu) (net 2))
 (segment (start 157.48 96.52) (end 158.900001 97.940001) (width 1) (layer B.Cu) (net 2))
 (segment (start 174.3 88.59) (end 179.07 83.82) (width 1) (layer B.Cu) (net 2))
 (segment (start 168.91 88.59) (end 174.3 88.59) (width 1) (layer B.Cu) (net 2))
 (segment (start 170.410001 79.930001) (end 168.91 78.43) (width 1) (layer B.Cu) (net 2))
 (segment (start 170.410001 87.089999) (end 170.410001 79.930001) (width 1) (layer B.Cu) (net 2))
 (segment (start 168.91 88.59) (end 170.410001 87.089999) (width 1) (layer B.Cu) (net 2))
 (segment (start 132.08 78.74) (end 140.97 69.85) (width 1) (layer B.Cu) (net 3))
 (segment (start 156.21 69.85) (end 158.75 72.39) (width 1) (layer B.Cu) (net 3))
 (segment (start 140.97 69.85) (end 156.21 69.85) (width 1) (layer B.Cu) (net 3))
 (segment (start 166.37 74.93) (end 162.56 78.74) (width 1) (layer B.Cu) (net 3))
 (segment (start 168.91 74.93) (end 166.37 74.93) (width 1) (layer B.Cu) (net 3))
 (segment (start 158.75 74.93) (end 162.56 78.74) (width 1) (layer B.Cu) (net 3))
 (segment (start 158.75 72.39) (end 158.75 74.93) (width 1) (layer B.Cu) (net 3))
 (segment (start 151.13 80.01) (end 152.4 78.74) (width 1) (layer B.Cu) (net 4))
 (segment (start 143.51 80.01) (end 151.13 80.01) (width 1) (layer B.Cu) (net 4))
 (segment (start 156.21 74.93) (end 156.21 72.39) (width 1) (layer B.Cu) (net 4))
 (segment (start 152.4 78.74) (end 156.21 74.93) (width 1) (layer B.Cu) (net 4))
 (segment (start 150.299999 86.799999) (end 152.4 88.9) (width 1) (layer B.Cu) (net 4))
 (segment (start 150.299999 80.840001) (end 150.299999 86.799999) (width 1) (layer B.Cu) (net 4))
 (segment (start 152.4 78.74) (end 150.299999 80.840001) (width 1) (layer B.Cu) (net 4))
 (segment (start 156.21 77.47) (end 162.56 83.82) (width 1) (layer B.Cu) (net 4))
 (segment (start 156.21 74.93) (end 156.21 77.47) (width 1) (layer B.Cu) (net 4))
 (segment (start 177.259999 76.929999) (end 179.07 78.74) (width 1) (layer B.Cu) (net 4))
 (segment (start 168.189999 76.929999) (end 177.259999 76.929999) (width 1) (layer B.Cu) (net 4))
 (segment (start 162.56 82.559998) (end 168.189999 76.929999) (width 1) (layer B.Cu) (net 4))
 (segment (start 162.56 83.82) (end 162.56 82.559998) (width 1) (layer B.Cu) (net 4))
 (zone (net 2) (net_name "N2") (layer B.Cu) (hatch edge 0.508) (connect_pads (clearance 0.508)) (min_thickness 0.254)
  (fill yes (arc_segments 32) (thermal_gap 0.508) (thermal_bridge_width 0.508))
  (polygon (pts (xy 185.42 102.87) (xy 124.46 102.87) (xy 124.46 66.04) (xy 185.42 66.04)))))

